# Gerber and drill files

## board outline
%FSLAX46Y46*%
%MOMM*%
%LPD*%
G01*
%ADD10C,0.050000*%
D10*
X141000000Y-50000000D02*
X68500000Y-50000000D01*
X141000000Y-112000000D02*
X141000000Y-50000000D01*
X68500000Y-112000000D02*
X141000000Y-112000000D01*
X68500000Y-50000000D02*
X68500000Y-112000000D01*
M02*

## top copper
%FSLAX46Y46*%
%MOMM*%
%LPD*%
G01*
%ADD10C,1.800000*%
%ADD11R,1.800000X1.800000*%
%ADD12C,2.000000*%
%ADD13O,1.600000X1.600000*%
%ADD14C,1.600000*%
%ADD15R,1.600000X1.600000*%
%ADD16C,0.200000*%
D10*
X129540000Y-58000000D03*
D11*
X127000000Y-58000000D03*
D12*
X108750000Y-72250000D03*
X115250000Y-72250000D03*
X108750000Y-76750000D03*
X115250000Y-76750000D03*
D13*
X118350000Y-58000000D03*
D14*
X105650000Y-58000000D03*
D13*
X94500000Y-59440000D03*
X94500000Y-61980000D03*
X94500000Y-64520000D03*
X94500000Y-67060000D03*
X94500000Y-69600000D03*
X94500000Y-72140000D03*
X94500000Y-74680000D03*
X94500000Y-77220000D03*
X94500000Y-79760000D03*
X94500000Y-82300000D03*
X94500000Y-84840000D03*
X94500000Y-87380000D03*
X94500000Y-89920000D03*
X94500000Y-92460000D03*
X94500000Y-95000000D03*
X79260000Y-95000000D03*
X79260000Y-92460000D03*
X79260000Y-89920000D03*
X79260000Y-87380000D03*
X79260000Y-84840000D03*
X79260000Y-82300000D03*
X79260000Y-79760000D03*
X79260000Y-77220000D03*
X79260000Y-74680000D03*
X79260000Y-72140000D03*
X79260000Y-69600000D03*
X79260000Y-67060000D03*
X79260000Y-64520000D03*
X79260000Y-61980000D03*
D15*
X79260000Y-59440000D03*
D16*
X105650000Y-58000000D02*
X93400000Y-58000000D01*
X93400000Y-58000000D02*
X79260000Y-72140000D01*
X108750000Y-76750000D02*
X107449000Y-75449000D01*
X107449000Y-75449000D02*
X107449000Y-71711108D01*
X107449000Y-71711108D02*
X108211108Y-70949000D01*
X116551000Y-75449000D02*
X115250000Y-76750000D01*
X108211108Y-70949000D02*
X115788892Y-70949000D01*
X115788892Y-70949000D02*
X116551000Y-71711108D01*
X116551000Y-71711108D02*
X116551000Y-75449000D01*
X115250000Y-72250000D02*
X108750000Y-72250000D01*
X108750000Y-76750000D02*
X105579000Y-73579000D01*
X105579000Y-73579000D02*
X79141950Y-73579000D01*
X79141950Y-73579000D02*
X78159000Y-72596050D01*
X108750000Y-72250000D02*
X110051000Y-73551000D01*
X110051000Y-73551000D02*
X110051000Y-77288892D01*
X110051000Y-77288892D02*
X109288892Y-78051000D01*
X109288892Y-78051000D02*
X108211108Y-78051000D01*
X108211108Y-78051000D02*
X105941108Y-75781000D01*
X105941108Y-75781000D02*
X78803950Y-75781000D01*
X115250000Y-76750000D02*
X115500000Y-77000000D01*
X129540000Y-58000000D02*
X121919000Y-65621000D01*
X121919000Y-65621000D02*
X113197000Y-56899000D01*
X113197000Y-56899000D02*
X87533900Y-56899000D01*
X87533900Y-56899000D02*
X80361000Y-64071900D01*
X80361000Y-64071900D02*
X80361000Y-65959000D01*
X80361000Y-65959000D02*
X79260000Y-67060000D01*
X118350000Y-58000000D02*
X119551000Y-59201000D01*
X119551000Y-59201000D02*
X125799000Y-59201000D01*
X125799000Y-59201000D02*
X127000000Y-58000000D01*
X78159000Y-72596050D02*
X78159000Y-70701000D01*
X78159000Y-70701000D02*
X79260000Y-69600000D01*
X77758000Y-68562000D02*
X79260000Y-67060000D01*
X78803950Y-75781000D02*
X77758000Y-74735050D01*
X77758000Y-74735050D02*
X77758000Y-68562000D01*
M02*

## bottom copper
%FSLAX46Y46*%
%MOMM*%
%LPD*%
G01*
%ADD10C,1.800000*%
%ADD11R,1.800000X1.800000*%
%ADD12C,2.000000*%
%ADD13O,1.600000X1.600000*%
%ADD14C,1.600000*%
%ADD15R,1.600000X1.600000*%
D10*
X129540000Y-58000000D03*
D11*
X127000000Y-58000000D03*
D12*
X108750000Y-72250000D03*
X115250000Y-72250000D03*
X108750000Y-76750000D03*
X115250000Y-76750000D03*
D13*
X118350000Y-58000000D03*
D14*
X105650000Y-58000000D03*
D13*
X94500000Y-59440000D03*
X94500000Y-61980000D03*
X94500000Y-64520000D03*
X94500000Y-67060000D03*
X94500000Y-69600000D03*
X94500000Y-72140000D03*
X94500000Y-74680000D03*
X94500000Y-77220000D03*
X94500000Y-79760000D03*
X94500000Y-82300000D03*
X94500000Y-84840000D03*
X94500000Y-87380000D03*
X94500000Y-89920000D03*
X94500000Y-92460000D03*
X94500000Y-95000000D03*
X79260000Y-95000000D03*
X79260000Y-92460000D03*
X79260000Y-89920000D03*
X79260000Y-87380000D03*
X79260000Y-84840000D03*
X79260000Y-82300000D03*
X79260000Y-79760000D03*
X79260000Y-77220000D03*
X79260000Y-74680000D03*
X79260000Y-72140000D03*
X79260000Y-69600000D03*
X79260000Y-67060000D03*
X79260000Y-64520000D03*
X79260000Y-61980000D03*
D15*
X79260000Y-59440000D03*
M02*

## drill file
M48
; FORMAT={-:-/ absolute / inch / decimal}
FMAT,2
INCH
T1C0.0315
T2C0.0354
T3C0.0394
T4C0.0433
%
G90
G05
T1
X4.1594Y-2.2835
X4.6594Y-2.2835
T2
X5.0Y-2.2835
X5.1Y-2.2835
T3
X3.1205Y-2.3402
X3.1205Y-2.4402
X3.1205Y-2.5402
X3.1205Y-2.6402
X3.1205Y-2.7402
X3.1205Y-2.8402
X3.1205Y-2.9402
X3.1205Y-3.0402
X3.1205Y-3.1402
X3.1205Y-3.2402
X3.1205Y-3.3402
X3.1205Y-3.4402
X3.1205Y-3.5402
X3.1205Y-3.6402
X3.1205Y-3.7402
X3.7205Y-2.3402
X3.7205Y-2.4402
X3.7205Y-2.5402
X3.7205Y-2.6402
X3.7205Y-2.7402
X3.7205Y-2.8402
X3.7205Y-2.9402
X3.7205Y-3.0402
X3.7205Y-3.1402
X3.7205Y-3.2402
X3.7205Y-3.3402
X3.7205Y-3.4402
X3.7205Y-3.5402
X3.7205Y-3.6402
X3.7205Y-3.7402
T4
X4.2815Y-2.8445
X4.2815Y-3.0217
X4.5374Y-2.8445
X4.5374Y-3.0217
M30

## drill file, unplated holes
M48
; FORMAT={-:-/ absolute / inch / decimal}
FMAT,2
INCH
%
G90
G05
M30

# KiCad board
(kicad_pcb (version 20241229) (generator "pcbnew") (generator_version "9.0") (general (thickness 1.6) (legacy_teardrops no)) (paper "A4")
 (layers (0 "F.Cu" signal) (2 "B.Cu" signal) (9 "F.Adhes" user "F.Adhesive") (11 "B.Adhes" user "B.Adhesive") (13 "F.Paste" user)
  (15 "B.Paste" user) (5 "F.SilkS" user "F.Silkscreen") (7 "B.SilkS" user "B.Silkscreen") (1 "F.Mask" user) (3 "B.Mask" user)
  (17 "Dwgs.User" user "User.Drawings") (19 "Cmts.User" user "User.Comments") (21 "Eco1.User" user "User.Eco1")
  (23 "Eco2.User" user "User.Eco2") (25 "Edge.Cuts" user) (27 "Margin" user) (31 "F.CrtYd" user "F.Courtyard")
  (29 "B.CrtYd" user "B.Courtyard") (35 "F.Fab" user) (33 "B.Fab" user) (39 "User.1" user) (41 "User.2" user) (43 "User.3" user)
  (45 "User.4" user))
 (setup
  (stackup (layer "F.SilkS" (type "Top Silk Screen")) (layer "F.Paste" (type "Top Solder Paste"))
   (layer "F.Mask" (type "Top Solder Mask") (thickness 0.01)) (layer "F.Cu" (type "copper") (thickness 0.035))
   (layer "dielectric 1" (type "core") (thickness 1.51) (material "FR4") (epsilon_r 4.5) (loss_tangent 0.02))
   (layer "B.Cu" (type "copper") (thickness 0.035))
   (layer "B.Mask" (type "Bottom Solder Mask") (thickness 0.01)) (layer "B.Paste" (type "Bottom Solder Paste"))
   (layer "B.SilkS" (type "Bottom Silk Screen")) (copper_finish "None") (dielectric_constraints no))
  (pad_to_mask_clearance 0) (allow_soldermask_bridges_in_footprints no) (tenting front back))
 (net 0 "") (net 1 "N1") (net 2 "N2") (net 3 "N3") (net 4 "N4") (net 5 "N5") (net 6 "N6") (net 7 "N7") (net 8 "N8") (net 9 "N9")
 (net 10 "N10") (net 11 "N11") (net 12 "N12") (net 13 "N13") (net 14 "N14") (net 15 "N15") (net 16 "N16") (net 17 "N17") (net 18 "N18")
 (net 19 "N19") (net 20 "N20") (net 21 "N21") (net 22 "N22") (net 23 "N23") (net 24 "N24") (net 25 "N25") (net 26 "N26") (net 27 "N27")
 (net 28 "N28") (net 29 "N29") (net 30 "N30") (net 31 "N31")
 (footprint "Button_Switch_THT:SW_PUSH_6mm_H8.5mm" (layer "F.Cu") (at 108.75 72.25)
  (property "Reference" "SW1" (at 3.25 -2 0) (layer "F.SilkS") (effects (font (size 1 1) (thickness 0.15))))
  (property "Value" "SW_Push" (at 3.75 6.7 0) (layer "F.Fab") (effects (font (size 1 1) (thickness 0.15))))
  (pad "1" thru_hole circle (at 0 0 90) (size 2 2) (drill 1.1) (layers "*.Cu" "*.Mask") (remove_unused_layers no) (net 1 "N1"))
  (pad "1" thru_hole circle (at 6.5 0 90) (size 2 2) (drill 1.1) (layers "*.Cu" "*.Mask") (remove_unused_layers no) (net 1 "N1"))
  (pad "2" thru_hole circle (at 0 4.5 90) (size 2 2) (drill 1.1) (layers "*.Cu" "*.Mask") (remove_unused_layers no) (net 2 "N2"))
  (pad "2" thru_hole circle (at 6.5 4.5 90) (size 2 2) (drill 1.1) (layers "*.Cu" "*.Mask") (remove_unused_layers no) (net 2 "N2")))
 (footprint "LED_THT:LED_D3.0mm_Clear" (layer "F.Cu") (at 127 58)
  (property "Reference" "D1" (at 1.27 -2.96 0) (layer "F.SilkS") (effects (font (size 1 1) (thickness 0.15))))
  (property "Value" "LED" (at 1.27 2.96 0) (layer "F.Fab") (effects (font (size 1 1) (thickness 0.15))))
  (pad "1" thru_hole rect (at 0 0) (size 1.8 1.8) (drill 0.9) (layers "*.Cu" "*.Mask") (remove_unused_layers no) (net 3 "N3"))
  (pad "2" thru_hole circle (at 2.54 0) (size 1.8 1.8) (drill 0.9) (layers "*.Cu" "*.Mask") (remove_unused_layers no) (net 1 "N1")))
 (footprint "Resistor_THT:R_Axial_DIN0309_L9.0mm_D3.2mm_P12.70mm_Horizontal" (layer "F.Cu") (at 105.65 58)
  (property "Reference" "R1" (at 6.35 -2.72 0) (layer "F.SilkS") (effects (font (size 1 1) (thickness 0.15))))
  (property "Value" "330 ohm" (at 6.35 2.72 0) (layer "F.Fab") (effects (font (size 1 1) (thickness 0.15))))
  (pad "1" thru_hole circle (at 0 0) (size 1.6 1.6) (drill 0.8) (layers "*.Cu" "*.Mask") (remove_unused_layers no) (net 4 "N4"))
  (pad "2" thru_hole oval (at 12.7 0) (size 1.6 1.6) (drill 0.8) (layers "*.Cu" "*.Mask") (remove_unused_layers no) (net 3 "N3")))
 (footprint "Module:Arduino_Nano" (layer "F.Cu") (at 79.26 59.44)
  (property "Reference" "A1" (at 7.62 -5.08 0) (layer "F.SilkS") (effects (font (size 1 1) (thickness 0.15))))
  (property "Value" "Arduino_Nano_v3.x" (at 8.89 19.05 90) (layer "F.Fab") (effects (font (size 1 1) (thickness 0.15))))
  (pad "1" thru_hole rect (at 0 0) (size 1.6 1.6) (drill 1) (layers "*.Cu" "*.Mask") (remove_unused_layers no) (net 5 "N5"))
  (pad "2" thru_hole oval (at 0 2.54) (size 1.6 1.6) (drill 1) (layers "*.Cu" "*.Mask") (remove_unused_layers no) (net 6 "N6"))
  (pad "3" thru_hole oval (at 0 5.08) (size 1.6 1.6) (drill 1) (layers "*.Cu" "*.Mask") (remove_unused_layers no) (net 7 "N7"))
  (pad "4" thru_hole oval (at 0 7.62) (size 1.6 1.6) (drill 1) (layers "*.Cu" "*.Mask") (remove_unused_layers no) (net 1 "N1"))
  (pad "5" thru_hole oval (at 0 10.16) (size 1.6 1.6) (drill 1) (layers "*.Cu" "*.Mask") (remove_unused_layers no) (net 2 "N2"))
  (pad "6" thru_hole oval (at 0 12.7) (size 1.6 1.6) (drill 1) (layers "*.Cu" "*.Mask") (remove_unused_layers no) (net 4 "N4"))
  (pad "7" thru_hole oval (at 0 15.24) (size 1.6 1.6) (drill 1) (layers "*.Cu" "*.Mask") (remove_unused_layers no) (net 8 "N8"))
  (pad "8" thru_hole oval (at 0 17.78) (size 1.6 1.6) (drill 1) (layers "*.Cu" "*.Mask") (remove_unused_layers no) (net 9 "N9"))
  (pad "9" thru_hole oval (at 0 20.32) (size 1.6 1.6) (drill 1) (layers "*.Cu" "*.Mask") (remove_unused_layers no) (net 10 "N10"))
  (pad "10" thru_hole oval (at 0 22.86) (size 1.6 1.6) (drill 1) (layers "*.Cu" "*.Mask") (remove_unused_layers no) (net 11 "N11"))
  (pad "11" thru_hole oval (at 0 25.4) (size 1.6 1.6) (drill 1) (layers "*.Cu" "*.Mask") (remove_unused_layers no) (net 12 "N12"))
  (pad "12" thru_hole oval (at 0 27.94) (size 1.6 1.6) (drill 1) (layers "*.Cu" "*.Mask") (remove_unused_layers no) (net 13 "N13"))
  (pad "13" thru_hole oval (at 0 30.48) (size 1.6 1.6) (drill 1) (layers "*.Cu" "*.Mask") (remove_unused_layers no) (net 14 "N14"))
  (pad "14" thru_hole oval (at 0 33.02) (size 1.6 1.6) (drill 1) (layers "*.Cu" "*.Mask") (remove_unused_layers no) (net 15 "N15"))
  (pad "15" thru_hole oval (at 0 35.56) (size 1.6 1.6) (drill 1) (layers "*.Cu" "*.Mask") (remove_unused_layers no) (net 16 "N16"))
  (pad "16" thru_hole oval (at 15.24 35.56) (size 1.6 1.6) (drill 1) (layers "*.Cu" "*.Mask") (remove_unused_layers no) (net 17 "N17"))
  (pad "17" thru_hole oval (at 15.24 33.02) (size 1.6 1.6) (drill 1) (layers "*.Cu" "*.Mask") (remove_unused_layers no) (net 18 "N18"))
  (pad "18" thru_hole oval (at 15.24 30.48) (size 1.6 1.6) (drill 1) (layers "*.Cu" "*.Mask") (remove_unused_layers no) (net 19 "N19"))
  (pad "19" thru_hole oval (at 15.24 27.94) (size 1.6 1.6) (drill 1) (layers "*.Cu" "*.Mask") (remove_unused_layers no) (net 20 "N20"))
  (pad "20" thru_hole oval (at 15.24 25.4) (size 1.6 1.6) (drill 1) (layers "*.Cu" "*.Mask") (remove_unused_layers no) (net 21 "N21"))
  (pad "21" thru_hole oval (at 15.24 22.86) (size 1.6 1.6) (drill 1) (layers "*.Cu" "*.Mask") (remove_unused_layers no) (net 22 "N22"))
  (pad "22" thru_hole oval (at 15.24 20.32) (size 1.6 1.6) (drill 1) (layers "*.Cu" "*.Mask") (remove_unused_layers no) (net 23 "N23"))
  (pad "23" thru_hole oval (at 15.24 17.78) (size 1.6 1.6) (drill 1) (layers "*.Cu" "*.Mask") (remove_unused_layers no) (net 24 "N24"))
  (pad "24" thru_hole oval (at 15.24 15.24) (size 1.6 1.6) (drill 1) (layers "*.Cu" "*.Mask") (remove_unused_layers no) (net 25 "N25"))
  (pad "25" thru_hole oval (at 15.24 12.7) (size 1.6 1.6) (drill 1) (layers "*.Cu" "*.Mask") (remove_unused_layers no) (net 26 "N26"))
  (pad "26" thru_hole oval (at 15.24 10.16) (size 1.6 1.6) (drill 1) (layers "*.Cu" "*.Mask") (remove_unused_layers no) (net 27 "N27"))
  (pad "27" thru_hole oval (at 15.24 7.62) (size 1.6 1.6) (drill 1) (layers "*.Cu" "*.Mask") (remove_unused_layers no) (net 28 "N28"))
  (pad "28" thru_hole oval (at 15.24 5.08) (size 1.6 1.6) (drill 1) (layers "*.Cu" "*.Mask") (remove_unused_layers no) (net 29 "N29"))
  (pad "29" thru_hole oval (at 15.24 2.54) (size 1.6 1.6) (drill 1) (layers "*.Cu" "*.Mask") (remove_unused_layers no) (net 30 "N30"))
  (pad "30" thru_hole oval (at 15.24 0) (size 1.6 1.6) (drill 1) (layers "*.Cu" "*.Mask") (remove_unused_layers no) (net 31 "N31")))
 (gr_line (start 68.5 50) (end 68.5 112) (stroke (width 0.05) (type default)) (layer "Edge.Cuts"))
 (gr_line (start 141 50) (end 68.5 50) (stroke (width 0.05) (type default)) (layer "Edge.Cuts"))
 (gr_line (start 68.5 112) (end 141 112) (stroke (width 0.05) (type default)) (layer "Edge.Cuts"))
 (gr_line (start 141 112) (end 141 50) (stroke (width 0.05) (type default)) (layer "Edge.Cuts"))
 (segment (start 93.4 58) (end 79.26 72.14) (width 0.2) (layer "F.Cu") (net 4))
 (segment (start 105.65 58) (end 93.4 58) (width 0.2) (layer "F.Cu") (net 4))
 (segment (start 105.579 73.579) (end 79.14195 73.579) (width 0.2) (layer "F.Cu") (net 2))
 (segment (start 108.211108 70.949) (end 115.788892 70.949) (width 0.2) (layer "F.Cu") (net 2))
 (segment (start 108.75 76.75) (end 105.579 73.579) (width 0.2) (layer "F.Cu") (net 2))
 (segment (start 78.159 72.59605) (end 78.159 70.701) (width 0.2) (layer "F.Cu") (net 2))
 (segment (start 107.449 75.449) (end 107.449 71.711108) (width 0.2) (layer "F.Cu") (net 2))
 (segment (start 108.75 76.75) (end 107.449 75.449) (width 0.2) (layer "F.Cu") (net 2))
 (segment (start 107.449 71.711108) (end 108.211108 70.949) (width 0.2) (layer "F.Cu") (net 2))
 (segment (start 115.25 76.75) (end 115.5 77) (width 0.2) (layer "F.Cu") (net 2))
 (segment (start 115.788892 70.949) (end 116.551 71.711108) (width 0.2) (layer "F.Cu") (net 2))
 (segment (start 116.551 75.449) (end 115.25 76.75) (width 0.2) (layer "F.Cu") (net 2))
 (segment (start 79.14195 73.579) (end 78.159 72.59605) (width 0.2) (layer "F.Cu") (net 2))
 (segment (start 78.159 70.701) (end 79.26 69.6) (width 0.2) (layer "F.Cu") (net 2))
 (segment (start 116.551 71.711108) (end 116.551 75.449) (width 0.2) (layer "F.Cu") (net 2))
 (segment (start 119.551 59.201) (end 125.799 59.201) (width 0.2) (layer "F.Cu") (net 3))
 (segment (start 118.35 58) (end 119.551 59.201) (width 0.2) (layer "F.Cu") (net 3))
 (segment (start 125.799 59.201) (end 127 58) (width 0.2) (layer "F.Cu") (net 3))
 (segment (start 113.197 56.899) (end 87.5339 56.899) (width 0.2) (layer "F.Cu") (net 1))
 (segment (start 80.361 65.959) (end 79.26 67.06) (width 0.2) (locked yes) (layer "F.Cu") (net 1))
 (segment (start 87.5339 56.899) (end 80.361 64.0719) (width 0.2) (layer "F.Cu") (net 1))
 (segment (start 77.758 68.562) (end 79.26 67.06) (width 0.2) (layer "F.Cu") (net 1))
 (segment (start 108.211108 78.051) (end 105.941108 75.781) (width 0.2) (layer "F.Cu") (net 1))
 (segment (start 121.919 65.621) (end 113.197 56.899) (width 0.2) (layer "F.Cu") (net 1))
 (segment (start 115.25 72.25) (end 108.75 72.25) (width 0.2) (layer "F.Cu") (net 1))
 (segment (start 110.051 73.551) (end 110.051 77.288892) (width 0.2) (layer "F.Cu") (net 1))
 (segment (start 80.361 64.0719) (end 80.361 65.959) (width 0.2) (layer "F.Cu") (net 1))
 (segment (start 105.941108 75.781) (end 78.80395 75.781) (width 0.2) (layer "F.Cu") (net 1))
 (segment (start 109.288892 78.051) (end 108.211108 78.051) (width 0.2) (layer "F.Cu") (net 1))
 (segment (start 77.758 74.73505) (end 77.758 68.562) (width 0.2) (layer "F.Cu") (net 1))
 (segment (start 129.54 58) (end 121.919 65.621) (width 0.2) (layer "F.Cu") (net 1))
 (segment (start 108.75 72.25) (end 110.051 73.551) (width 0.2) (layer "F.Cu") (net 1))
 (segment (start 110.051 77.288892) (end 109.288892 78.051) (width 0.2) (layer "F.Cu") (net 1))
 (segment (start 78.80395 75.781) (end 77.758 74.73505) (width 0.2) (layer "F.Cu") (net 1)))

